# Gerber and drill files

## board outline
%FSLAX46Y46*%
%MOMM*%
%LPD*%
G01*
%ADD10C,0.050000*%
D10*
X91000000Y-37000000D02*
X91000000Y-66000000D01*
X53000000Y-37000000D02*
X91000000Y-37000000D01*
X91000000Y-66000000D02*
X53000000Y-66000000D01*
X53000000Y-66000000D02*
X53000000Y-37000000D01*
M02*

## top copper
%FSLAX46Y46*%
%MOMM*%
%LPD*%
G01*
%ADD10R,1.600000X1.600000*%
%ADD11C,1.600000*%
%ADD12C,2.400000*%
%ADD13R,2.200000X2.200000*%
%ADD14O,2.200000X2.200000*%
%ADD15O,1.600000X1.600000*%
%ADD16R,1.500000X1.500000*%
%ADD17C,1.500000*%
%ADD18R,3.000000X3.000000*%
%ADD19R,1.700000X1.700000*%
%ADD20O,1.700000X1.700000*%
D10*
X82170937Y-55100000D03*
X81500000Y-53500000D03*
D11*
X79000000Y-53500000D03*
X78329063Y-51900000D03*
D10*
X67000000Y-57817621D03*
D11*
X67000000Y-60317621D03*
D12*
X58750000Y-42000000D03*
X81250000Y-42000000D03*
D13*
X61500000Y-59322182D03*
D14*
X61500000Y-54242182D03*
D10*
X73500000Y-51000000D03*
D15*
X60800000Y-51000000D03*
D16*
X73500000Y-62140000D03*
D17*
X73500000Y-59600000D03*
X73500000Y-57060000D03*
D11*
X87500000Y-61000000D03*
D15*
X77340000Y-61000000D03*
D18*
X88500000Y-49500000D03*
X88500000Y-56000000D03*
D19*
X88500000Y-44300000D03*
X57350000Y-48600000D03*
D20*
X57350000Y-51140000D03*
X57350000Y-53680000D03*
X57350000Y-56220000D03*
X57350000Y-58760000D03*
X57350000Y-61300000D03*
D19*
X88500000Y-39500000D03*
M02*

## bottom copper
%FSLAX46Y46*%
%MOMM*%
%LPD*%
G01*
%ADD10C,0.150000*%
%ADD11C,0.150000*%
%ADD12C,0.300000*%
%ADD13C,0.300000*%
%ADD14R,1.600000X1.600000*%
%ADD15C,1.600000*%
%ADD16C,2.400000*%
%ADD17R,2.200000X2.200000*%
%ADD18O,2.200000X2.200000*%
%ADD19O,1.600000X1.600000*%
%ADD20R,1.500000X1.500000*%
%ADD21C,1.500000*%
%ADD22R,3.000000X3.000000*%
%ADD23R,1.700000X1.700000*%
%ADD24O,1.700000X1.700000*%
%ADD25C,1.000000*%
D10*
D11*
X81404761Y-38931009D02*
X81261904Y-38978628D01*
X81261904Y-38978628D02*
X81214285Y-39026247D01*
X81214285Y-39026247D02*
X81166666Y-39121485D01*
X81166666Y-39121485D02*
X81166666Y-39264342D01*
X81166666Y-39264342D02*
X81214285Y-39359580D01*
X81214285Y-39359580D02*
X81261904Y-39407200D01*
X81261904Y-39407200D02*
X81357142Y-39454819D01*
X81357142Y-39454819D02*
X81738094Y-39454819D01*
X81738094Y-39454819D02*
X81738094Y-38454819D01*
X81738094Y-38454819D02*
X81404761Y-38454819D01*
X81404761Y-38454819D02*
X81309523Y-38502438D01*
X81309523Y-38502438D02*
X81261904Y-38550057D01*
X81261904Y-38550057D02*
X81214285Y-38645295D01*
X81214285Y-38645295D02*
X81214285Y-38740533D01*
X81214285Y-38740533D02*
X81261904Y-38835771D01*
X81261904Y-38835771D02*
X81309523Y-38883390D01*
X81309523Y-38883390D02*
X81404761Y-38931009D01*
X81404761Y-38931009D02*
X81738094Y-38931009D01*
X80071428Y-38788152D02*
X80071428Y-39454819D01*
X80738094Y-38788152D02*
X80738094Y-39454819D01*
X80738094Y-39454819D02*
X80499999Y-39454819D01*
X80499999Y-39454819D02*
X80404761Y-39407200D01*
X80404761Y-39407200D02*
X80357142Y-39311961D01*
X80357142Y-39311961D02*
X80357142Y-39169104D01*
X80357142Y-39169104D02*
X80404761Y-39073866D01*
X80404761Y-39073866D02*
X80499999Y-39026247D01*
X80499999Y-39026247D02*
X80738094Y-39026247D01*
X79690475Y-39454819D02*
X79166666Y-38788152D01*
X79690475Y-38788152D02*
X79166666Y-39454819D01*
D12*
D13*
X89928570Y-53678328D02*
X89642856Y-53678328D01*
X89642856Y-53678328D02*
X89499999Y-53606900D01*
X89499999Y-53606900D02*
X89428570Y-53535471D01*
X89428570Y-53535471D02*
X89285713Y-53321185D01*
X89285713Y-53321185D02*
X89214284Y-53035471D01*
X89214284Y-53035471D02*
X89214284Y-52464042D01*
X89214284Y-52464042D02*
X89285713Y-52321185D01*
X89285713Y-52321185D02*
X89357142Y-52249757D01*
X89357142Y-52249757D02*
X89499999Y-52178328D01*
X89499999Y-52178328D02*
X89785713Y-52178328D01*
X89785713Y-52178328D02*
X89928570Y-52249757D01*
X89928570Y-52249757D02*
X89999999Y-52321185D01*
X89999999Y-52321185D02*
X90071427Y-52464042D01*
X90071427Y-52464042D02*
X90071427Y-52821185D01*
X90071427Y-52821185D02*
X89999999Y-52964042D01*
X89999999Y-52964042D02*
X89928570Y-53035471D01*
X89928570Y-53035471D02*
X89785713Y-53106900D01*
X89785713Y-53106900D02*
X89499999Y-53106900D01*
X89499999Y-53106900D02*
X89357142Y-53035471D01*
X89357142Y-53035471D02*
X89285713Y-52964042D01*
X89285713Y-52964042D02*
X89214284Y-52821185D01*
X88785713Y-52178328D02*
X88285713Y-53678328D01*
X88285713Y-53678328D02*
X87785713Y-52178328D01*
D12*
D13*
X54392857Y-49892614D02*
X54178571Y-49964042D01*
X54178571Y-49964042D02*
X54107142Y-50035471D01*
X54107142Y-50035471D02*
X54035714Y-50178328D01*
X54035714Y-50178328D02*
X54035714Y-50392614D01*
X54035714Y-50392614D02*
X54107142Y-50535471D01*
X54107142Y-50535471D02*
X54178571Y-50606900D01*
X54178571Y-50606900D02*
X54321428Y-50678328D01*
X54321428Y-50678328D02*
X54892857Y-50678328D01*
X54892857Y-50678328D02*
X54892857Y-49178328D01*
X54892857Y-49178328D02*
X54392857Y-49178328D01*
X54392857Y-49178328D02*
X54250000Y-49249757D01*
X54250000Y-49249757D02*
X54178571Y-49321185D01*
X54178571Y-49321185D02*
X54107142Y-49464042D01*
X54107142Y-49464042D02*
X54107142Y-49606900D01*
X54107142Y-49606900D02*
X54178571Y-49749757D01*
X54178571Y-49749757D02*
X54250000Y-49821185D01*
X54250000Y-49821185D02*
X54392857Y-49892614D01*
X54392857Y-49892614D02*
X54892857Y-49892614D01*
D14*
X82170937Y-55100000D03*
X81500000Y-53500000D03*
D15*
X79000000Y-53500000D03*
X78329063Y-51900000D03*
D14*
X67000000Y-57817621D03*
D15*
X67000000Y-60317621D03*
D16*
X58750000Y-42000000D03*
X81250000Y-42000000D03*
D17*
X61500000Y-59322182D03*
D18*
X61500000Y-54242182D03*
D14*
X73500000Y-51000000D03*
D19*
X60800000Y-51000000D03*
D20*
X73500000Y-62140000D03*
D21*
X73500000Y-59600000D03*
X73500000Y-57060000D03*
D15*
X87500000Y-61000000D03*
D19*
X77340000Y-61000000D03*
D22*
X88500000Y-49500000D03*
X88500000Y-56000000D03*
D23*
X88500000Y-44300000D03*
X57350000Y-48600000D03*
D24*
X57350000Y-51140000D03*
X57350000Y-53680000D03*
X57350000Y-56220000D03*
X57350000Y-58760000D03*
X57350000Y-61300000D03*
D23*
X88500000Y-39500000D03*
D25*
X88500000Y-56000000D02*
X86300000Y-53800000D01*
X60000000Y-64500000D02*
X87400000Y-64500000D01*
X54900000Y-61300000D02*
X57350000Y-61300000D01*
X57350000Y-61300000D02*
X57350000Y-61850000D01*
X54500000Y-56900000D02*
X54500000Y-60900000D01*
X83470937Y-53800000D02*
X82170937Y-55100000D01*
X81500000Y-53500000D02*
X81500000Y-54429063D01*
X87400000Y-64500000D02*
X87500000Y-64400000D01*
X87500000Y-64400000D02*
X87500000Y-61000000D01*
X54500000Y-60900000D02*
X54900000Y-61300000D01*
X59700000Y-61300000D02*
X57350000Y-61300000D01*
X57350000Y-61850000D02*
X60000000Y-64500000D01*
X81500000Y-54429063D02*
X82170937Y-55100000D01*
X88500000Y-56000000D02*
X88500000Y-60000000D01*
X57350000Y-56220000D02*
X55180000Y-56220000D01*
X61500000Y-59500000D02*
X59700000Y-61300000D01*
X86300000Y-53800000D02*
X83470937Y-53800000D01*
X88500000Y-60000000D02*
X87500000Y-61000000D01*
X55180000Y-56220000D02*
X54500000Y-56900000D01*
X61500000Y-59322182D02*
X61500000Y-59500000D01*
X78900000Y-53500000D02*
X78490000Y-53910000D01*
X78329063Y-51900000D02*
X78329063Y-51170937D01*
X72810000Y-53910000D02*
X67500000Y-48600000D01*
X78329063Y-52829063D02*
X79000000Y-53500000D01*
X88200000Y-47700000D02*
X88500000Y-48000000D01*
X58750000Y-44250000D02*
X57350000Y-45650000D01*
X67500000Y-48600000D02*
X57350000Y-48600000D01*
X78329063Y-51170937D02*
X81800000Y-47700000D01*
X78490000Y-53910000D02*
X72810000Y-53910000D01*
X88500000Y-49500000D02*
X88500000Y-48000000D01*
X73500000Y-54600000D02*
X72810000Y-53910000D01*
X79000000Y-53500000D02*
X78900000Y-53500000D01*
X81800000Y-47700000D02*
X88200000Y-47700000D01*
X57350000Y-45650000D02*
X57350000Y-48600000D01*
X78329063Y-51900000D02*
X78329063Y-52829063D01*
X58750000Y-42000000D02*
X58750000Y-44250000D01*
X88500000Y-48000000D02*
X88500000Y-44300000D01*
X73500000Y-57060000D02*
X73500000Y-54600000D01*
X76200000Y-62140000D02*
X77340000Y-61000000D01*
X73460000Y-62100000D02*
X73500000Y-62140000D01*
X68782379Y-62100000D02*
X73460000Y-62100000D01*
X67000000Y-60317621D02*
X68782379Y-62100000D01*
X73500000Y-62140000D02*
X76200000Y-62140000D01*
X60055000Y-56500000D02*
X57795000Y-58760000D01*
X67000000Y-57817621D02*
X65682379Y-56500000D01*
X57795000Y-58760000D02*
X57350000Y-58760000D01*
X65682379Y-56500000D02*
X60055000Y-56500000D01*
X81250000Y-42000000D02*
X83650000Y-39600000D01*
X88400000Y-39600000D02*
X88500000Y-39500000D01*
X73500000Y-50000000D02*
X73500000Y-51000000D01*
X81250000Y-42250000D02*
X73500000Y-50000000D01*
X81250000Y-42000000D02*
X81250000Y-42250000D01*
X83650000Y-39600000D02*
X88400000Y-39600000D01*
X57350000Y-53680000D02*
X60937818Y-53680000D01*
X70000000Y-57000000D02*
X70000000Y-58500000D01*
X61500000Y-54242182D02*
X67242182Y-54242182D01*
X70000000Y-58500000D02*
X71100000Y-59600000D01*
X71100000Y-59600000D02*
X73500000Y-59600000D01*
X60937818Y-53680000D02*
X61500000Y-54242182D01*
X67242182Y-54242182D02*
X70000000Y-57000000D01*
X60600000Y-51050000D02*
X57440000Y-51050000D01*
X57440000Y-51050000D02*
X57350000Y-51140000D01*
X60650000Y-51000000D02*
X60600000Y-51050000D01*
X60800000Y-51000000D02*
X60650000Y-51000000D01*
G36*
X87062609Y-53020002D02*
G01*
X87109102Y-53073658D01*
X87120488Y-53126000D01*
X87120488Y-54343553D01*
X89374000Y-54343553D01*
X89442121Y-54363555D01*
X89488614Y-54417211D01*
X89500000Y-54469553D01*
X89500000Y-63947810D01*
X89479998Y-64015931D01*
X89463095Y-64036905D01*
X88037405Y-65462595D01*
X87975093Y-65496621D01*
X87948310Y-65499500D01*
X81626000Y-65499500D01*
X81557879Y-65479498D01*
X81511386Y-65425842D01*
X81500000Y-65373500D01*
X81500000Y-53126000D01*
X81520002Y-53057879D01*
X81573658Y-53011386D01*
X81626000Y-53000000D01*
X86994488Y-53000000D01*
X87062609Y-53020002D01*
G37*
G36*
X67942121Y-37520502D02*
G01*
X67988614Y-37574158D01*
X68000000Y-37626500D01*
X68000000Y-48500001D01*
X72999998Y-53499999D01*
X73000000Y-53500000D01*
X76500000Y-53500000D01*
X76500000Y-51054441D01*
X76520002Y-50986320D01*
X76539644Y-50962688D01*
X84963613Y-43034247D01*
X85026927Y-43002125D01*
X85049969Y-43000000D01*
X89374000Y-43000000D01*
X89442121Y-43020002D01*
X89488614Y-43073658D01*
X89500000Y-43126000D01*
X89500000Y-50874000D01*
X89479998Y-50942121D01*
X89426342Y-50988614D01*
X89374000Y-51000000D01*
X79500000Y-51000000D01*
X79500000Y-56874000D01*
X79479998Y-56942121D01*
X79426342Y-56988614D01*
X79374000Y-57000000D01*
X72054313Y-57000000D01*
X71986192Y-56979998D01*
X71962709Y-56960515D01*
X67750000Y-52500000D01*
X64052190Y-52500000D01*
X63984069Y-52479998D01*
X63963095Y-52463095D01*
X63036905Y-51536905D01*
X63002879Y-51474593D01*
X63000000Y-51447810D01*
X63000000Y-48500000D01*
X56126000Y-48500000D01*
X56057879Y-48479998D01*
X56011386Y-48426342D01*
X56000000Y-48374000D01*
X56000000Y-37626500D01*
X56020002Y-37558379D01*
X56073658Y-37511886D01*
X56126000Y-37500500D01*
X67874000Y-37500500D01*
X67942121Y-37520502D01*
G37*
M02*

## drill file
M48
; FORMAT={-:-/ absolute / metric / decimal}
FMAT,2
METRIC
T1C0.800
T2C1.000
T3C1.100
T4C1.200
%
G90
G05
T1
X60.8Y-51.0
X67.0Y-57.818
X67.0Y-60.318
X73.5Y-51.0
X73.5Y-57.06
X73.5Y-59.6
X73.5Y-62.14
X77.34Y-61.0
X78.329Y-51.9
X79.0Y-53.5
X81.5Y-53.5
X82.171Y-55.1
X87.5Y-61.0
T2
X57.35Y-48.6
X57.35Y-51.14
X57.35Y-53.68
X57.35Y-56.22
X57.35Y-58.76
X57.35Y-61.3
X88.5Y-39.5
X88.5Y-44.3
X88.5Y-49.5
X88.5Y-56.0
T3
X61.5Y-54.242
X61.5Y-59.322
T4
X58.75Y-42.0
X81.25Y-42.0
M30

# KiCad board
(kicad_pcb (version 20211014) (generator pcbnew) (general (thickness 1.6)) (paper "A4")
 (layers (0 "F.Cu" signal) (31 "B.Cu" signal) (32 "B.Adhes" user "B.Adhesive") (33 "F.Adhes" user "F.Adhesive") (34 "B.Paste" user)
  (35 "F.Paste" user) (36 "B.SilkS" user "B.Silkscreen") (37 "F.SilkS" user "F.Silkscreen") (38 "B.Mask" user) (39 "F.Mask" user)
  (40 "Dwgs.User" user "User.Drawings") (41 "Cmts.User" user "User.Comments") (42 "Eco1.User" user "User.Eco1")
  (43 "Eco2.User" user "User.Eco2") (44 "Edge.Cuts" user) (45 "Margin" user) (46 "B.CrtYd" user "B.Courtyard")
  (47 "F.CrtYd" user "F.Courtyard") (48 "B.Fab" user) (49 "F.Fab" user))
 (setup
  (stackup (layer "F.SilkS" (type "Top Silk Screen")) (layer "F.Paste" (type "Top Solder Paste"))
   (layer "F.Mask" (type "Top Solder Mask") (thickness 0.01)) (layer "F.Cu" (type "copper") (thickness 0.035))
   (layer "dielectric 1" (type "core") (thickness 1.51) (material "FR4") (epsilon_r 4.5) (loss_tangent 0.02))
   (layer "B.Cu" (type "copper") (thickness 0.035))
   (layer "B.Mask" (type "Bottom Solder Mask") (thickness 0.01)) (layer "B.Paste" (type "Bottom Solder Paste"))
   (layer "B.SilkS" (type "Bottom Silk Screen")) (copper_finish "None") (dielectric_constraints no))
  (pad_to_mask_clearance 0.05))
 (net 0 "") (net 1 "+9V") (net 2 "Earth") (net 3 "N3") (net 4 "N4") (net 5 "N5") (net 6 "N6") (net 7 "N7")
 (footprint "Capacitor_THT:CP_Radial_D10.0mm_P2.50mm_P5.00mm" (layer "F.Cu") (at 81.5 53.5 180)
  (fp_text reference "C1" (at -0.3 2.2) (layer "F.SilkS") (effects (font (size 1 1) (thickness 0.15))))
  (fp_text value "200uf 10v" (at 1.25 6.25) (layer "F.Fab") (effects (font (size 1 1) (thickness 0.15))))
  (pad "1" thru_hole rect locked (at -0.670937 -1.6 180) (size 1.6 1.6) (drill 0.8) (layers *.Cu *.Mask) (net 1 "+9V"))
  (pad "1" thru_hole rect locked (at 0 0 180) (size 1.6 1.6) (drill 0.8) (layers *.Cu *.Mask) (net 1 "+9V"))
  (pad "2" thru_hole circle locked (at 2.5 0 180) (size 1.6 1.6) (drill 0.8) (layers *.Cu *.Mask) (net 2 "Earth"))
  (pad "2" thru_hole circle locked (at 3.170937 1.6 180) (size 1.6 1.6) (drill 0.8) (layers *.Cu *.Mask) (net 2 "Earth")))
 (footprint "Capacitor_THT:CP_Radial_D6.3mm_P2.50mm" (layer "F.Cu") (at 67 57.817621 -90)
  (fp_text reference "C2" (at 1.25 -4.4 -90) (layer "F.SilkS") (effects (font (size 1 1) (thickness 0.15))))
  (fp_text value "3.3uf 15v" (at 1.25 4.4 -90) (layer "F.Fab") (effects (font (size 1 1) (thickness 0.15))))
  (pad "1" thru_hole rect locked (at 0 0 270) (size 1.6 1.6) (drill 0.8) (layers *.Cu *.Mask) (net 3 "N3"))
  (pad "2" thru_hole circle locked (at 2.5 0 270) (size 1.6 1.6) (drill 0.8) (layers *.Cu *.Mask) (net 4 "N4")))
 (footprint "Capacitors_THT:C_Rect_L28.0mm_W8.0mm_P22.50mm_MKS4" (layer "F.Cu") (at 58.75 42)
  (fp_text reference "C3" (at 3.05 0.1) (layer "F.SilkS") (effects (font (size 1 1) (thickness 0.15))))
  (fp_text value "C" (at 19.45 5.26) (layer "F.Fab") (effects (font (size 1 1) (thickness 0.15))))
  (pad "1" thru_hole circle locked (at 0 0) (size 2.4 2.4) (drill 1.2) (layers *.Cu *.Mask) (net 2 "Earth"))
  (pad "2" thru_hole circle locked (at 22.5 0) (size 2.4 2.4) (drill 1.2) (layers *.Cu *.Mask) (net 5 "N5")))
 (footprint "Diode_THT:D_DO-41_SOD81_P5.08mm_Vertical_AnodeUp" (layer "F.Cu") (at 61.5 59.322182 90)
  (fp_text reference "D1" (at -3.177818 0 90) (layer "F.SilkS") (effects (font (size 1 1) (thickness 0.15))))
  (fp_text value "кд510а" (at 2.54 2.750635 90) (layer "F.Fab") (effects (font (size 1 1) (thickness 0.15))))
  (pad "1" thru_hole rect locked (at 0 0 90) (size 2.2 2.2) (drill 1.1) (layers *.Cu *.Mask) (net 1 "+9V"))
  (pad "2" thru_hole oval locked (at 5.08 0 90) (size 2.2 2.2) (drill 1.1) (layers *.Cu *.Mask) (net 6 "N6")))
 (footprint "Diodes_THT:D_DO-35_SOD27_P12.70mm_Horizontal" (layer "F.Cu") (at 73.5 51 180)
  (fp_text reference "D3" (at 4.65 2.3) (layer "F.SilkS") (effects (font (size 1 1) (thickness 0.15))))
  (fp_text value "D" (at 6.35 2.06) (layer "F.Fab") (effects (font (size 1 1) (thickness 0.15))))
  (pad "1" thru_hole rect locked (at 0 0 180) (size 1.6 1.6) (drill 0.8) (layers *.Cu *.Mask) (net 5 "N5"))
  (pad "2" thru_hole oval locked (at 12.7 0 180) (size 1.6 1.6) (drill 0.8) (layers *.Cu *.Mask) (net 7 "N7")))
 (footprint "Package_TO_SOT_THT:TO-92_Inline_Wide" (layer "F.Cu") (at 73.5 62.14 90)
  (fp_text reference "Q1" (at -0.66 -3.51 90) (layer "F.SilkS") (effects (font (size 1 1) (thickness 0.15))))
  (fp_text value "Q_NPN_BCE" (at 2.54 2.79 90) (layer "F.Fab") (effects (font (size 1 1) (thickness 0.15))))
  (pad "1" thru_hole rect locked (at 0 0 90) (size 1.5 1.5) (drill 0.8) (layers *.Cu *.Mask) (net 4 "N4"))
  (pad "2" thru_hole circle locked (at 2.54 0 90) (size 1.5 1.5) (drill 0.8) (layers *.Cu *.Mask) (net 6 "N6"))
  (pad "3" thru_hole circle locked (at 5.08 0 90) (size 1.5 1.5) (drill 0.8) (layers *.Cu *.Mask) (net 2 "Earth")))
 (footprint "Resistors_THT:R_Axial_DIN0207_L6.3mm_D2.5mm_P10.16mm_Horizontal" (layer "F.Cu") (at 87.5 61 180)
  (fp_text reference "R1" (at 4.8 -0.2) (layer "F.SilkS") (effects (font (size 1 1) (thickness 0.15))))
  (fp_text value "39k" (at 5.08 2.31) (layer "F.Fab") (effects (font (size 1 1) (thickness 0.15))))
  (pad "1" thru_hole circle locked (at 0 0 180) (size 1.6 1.6) (drill 0.8) (layers *.Cu *.Mask) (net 1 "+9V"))
  (pad "2" thru_hole oval locked (at 10.16 0 180) (size 1.6 1.6) (drill 0.8) (layers *.Cu *.Mask) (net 4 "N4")))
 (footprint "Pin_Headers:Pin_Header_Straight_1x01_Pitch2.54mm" (layer "F.Cu") (at 88.5 49.5 90)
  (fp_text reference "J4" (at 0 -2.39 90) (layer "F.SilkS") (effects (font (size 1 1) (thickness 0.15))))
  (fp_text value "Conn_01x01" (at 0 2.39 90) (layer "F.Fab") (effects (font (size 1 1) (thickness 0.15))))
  (pad "1" thru_hole rect locked (at 0 0 90) (size 3 3) (drill 1) (layers *.Cu *.Mask) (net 2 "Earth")))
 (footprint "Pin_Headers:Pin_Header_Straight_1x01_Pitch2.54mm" (layer "F.Cu") (at 88.5 56 90)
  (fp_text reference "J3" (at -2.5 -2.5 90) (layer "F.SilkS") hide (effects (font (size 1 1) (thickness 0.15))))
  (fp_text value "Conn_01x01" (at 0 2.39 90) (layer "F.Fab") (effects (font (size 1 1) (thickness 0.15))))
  (pad "1" thru_hole rect locked (at 0 0 90) (size 3 3) (drill 1) (layers *.Cu *.Mask) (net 1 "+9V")))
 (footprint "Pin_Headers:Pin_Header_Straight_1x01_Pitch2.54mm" (layer "F.Cu") (at 88.5 44.3)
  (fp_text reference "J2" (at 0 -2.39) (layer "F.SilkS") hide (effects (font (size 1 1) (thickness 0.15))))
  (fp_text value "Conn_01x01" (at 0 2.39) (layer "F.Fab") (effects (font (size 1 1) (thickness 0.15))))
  (pad "1" thru_hole rect locked (at 0 0) (size 1.7 1.7) (drill 1) (layers *.Cu *.Mask) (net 2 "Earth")))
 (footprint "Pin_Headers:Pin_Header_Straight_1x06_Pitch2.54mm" (layer "F.Cu") (at 57.35 48.6)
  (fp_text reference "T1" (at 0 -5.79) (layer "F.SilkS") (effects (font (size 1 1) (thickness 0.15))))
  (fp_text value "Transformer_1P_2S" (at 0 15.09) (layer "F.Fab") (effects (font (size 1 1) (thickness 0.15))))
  (pad "1" thru_hole rect locked (at 0 0) (size 1.7 1.7) (drill 1) (layers *.Cu *.Mask) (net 2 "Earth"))
  (pad "2" thru_hole oval locked (at 0 2.54) (size 1.7 1.7) (drill 1) (layers *.Cu *.Mask) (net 7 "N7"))
  (pad "3" thru_hole oval locked (at 0 5.08) (size 1.7 1.7) (drill 1) (layers *.Cu *.Mask) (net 6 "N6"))
  (pad "4" thru_hole oval locked (at 0 7.62) (size 1.7 1.7) (drill 1) (layers *.Cu *.Mask) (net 1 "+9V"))
  (pad "5" thru_hole oval locked (at 0 10.16) (size 1.7 1.7) (drill 1) (layers *.Cu *.Mask) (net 3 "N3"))
  (pad "6" thru_hole oval locked (at 0 12.7) (size 1.7 1.7) (drill 1) (layers *.Cu *.Mask) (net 1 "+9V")))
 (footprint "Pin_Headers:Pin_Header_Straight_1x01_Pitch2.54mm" (layer "F.Cu") (at 88.5 39.5)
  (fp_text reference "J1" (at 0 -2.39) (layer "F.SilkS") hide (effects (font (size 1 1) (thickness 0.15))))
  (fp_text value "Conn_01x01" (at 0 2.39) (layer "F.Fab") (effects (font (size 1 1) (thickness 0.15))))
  (pad "1" thru_hole rect locked (at 0 0) (size 1.7 1.7) (drill 1) (layers *.Cu *.Mask) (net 5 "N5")))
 (gr_line (start 91 37) (end 91 66) (layer "Edge.Cuts") (width 0.05))
 (gr_line (start 53 37) (end 91 37) (layer "Edge.Cuts") (width 0.05))
 (gr_line (start 91 66) (end 53 66) (layer "Edge.Cuts") (width 0.05))
 (gr_line (start 53 66) (end 53 37) (layer "Edge.Cuts") (width 0.05))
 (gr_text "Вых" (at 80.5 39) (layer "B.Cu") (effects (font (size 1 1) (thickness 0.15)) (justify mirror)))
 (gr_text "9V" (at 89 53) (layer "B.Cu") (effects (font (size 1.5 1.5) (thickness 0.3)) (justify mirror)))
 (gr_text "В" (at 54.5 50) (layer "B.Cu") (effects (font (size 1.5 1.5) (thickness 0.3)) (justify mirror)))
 (segment (start 88.5 56) (end 86.3 53.8) (width 1) (layer "B.Cu") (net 1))
 (segment (start 60 64.5) (end 87.4 64.5) (width 1) (layer "B.Cu") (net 1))
 (segment (start 54.9 61.3) (end 57.35 61.3) (width 1) (layer "B.Cu") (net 1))
 (segment (start 57.35 61.3) (end 57.35 61.85) (width 1) (layer "B.Cu") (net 1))
 (segment (start 54.5 56.9) (end 54.5 60.9) (width 1) (layer "B.Cu") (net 1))
 (segment (start 83.470937 53.8) (end 82.170937 55.1) (width 1) (layer "B.Cu") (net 1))
 (segment (start 81.5 53.5) (end 81.5 54.429063) (width 1) (layer "B.Cu") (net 1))
 (segment (start 87.4 64.5) (end 87.5 64.4) (width 1) (layer "B.Cu") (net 1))
 (segment (start 87.5 64.4) (end 87.5 61) (width 1) (layer "B.Cu") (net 1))
 (segment (start 54.5 60.9) (end 54.9 61.3) (width 1) (layer "B.Cu") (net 1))
 (segment (start 59.7 61.3) (end 57.35 61.3) (width 1) (layer "B.Cu") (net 1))
 (segment (start 57.35 61.85) (end 60 64.5) (width 1) (layer "B.Cu") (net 1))
 (segment (start 81.5 54.429063) (end 82.170937 55.1) (width 1) (layer "B.Cu") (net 1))
 (segment (start 88.5 56) (end 88.5 60) (width 1) (layer "B.Cu") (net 1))
 (segment (start 57.35 56.22) (end 55.18 56.22) (width 1) (layer "B.Cu") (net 1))
 (segment (start 61.5 59.5) (end 59.7 61.3) (width 1) (layer "B.Cu") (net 1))
 (segment (start 86.3 53.8) (end 83.470937 53.8) (width 1) (layer "B.Cu") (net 1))
 (segment (start 88.5 60) (end 87.5 61) (width 1) (layer "B.Cu") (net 1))
 (segment (start 55.18 56.22) (end 54.5 56.9) (width 1) (layer "B.Cu") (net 1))
 (segment (start 61.5 59.322182) (end 61.5 59.5) (width 1) (layer "B.Cu") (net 1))
 (segment (start 78.9 53.5) (end 78.49 53.91) (width 1) (layer "B.Cu") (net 2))
 (segment (start 78.329063 51.9) (end 78.329063 51.170937) (width 1) (layer "B.Cu") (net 2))
 (segment (start 72.81 53.91) (end 67.5 48.6) (width 1) (layer "B.Cu") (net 2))
 (segment (start 78.329063 52.829063) (end 79 53.5) (width 1) (layer "B.Cu") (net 2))
 (segment (start 88.2 47.7) (end 88.5 48) (width 1) (layer "B.Cu") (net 2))
 (segment (start 58.75 44.25) (end 57.35 45.65) (width 1) (layer "B.Cu") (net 2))
 (segment (start 67.5 48.6) (end 57.35 48.6) (width 1) (layer "B.Cu") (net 2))
 (segment (start 78.329063 51.170937) (end 81.8 47.7) (width 1) (layer "B.Cu") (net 2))
 (segment (start 78.49 53.91) (end 72.81 53.91) (width 1) (layer "B.Cu") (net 2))
 (segment (start 88.5 49.5) (end 88.5 48) (width 1) (layer "B.Cu") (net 2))
 (segment (start 73.5 54.6) (end 72.81 53.91) (width 1) (layer "B.Cu") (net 2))
 (segment (start 79 53.5) (end 78.9 53.5) (width 1) (layer "B.Cu") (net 2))
 (segment (start 81.8 47.7) (end 88.2 47.7) (width 1) (layer "B.Cu") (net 2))
 (segment (start 57.35 45.65) (end 57.35 48.6) (width 1) (layer "B.Cu") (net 2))
 (segment (start 78.329063 51.9) (end 78.329063 52.829063) (width 1) (layer "B.Cu") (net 2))
 (segment (start 58.75 42) (end 58.75 44.25) (width 1) (layer "B.Cu") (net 2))
 (segment (start 88.5 48) (end 88.5 44.3) (width 1) (layer "B.Cu") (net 2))
 (segment (start 73.5 57.06) (end 73.5 54.6) (width 1) (layer "B.Cu") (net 2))
 (segment (start 76.2 62.14) (end 77.34 61) (width 1) (layer "B.Cu") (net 4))
 (segment (start 73.46 62.1) (end 73.5 62.14) (width 1) (layer "B.Cu") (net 4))
 (segment (start 68.782379 62.1) (end 73.46 62.1) (width 1) (layer "B.Cu") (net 4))
 (segment (start 67 60.317621) (end 68.782379 62.1) (width 1) (layer "B.Cu") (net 4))
 (segment (start 73.5 62.14) (end 76.2 62.14) (width 1) (layer "B.Cu") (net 4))
 (segment (start 60.055 56.5) (end 57.795 58.76) (width 1) (layer "B.Cu") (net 3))
 (segment (start 67 57.817621) (end 65.682379 56.5) (width 1) (layer "B.Cu") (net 3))
 (segment (start 57.795 58.76) (end 57.35 58.76) (width 1) (layer "B.Cu") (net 3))
 (segment (start 65.682379 56.5) (end 60.055 56.5) (width 1) (layer "B.Cu") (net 3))
 (segment (start 81.25 42) (end 83.65 39.6) (width 1) (layer "B.Cu") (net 5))
 (segment (start 88.4 39.6) (end 88.5 39.5) (width 1) (layer "B.Cu") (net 5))
 (segment (start 73.5 50) (end 73.5 51) (width 1) (layer "B.Cu") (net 5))
 (segment (start 81.25 42.25) (end 73.5 50) (width 1) (layer "B.Cu") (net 5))
 (segment (start 81.25 42) (end 81.25 42.25) (width 1) (layer "B.Cu") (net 5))
 (segment (start 83.65 39.6) (end 88.4 39.6) (width 1) (layer "B.Cu") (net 5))
 (segment (start 57.35 53.68) (end 60.937818 53.68) (width 1) (layer "B.Cu") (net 6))
 (segment (start 70 57) (end 70 58.5) (width 1) (layer "B.Cu") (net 6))
 (segment (start 61.5 54.242182) (end 67.242182 54.242182) (width 1) (layer "B.Cu") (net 6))
 (segment (start 70 58.5) (end 71.1 59.6) (width 1) (layer "B.Cu") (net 6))
 (segment (start 71.1 59.6) (end 73.5 59.6) (width 1) (layer "B.Cu") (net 6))
 (segment (start 60.937818 53.68) (end 61.5 54.242182) (width 1) (layer "B.Cu") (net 6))
 (segment (start 67.242182 54.242182) (end 70 57) (width 1) (layer "B.Cu") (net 6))
 (segment (start 60.6 51.05) (end 57.44 51.05) (width 1) (layer "B.Cu") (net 7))
 (segment (start 57.44 51.05) (end 57.35 51.14) (width 1) (layer "B.Cu") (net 7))
 (segment (start 60.65 51) (end 60.6 51.05) (width 1) (layer "B.Cu") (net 7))
 (segment (start 60.8 51) (end 60.65 51) (width 1) (layer "B.Cu") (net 7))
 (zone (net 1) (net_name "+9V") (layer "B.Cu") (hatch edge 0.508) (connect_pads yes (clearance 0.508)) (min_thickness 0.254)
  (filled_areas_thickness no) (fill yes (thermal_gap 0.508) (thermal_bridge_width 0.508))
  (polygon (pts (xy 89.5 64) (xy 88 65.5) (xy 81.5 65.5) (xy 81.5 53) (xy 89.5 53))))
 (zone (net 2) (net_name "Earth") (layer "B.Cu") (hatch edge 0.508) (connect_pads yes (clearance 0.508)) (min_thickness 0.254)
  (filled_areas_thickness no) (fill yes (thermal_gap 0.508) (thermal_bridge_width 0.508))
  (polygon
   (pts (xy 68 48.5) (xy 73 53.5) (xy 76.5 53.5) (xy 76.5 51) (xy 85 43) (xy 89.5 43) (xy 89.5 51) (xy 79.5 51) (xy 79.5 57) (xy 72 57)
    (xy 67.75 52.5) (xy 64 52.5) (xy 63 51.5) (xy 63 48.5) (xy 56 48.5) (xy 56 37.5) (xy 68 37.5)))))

